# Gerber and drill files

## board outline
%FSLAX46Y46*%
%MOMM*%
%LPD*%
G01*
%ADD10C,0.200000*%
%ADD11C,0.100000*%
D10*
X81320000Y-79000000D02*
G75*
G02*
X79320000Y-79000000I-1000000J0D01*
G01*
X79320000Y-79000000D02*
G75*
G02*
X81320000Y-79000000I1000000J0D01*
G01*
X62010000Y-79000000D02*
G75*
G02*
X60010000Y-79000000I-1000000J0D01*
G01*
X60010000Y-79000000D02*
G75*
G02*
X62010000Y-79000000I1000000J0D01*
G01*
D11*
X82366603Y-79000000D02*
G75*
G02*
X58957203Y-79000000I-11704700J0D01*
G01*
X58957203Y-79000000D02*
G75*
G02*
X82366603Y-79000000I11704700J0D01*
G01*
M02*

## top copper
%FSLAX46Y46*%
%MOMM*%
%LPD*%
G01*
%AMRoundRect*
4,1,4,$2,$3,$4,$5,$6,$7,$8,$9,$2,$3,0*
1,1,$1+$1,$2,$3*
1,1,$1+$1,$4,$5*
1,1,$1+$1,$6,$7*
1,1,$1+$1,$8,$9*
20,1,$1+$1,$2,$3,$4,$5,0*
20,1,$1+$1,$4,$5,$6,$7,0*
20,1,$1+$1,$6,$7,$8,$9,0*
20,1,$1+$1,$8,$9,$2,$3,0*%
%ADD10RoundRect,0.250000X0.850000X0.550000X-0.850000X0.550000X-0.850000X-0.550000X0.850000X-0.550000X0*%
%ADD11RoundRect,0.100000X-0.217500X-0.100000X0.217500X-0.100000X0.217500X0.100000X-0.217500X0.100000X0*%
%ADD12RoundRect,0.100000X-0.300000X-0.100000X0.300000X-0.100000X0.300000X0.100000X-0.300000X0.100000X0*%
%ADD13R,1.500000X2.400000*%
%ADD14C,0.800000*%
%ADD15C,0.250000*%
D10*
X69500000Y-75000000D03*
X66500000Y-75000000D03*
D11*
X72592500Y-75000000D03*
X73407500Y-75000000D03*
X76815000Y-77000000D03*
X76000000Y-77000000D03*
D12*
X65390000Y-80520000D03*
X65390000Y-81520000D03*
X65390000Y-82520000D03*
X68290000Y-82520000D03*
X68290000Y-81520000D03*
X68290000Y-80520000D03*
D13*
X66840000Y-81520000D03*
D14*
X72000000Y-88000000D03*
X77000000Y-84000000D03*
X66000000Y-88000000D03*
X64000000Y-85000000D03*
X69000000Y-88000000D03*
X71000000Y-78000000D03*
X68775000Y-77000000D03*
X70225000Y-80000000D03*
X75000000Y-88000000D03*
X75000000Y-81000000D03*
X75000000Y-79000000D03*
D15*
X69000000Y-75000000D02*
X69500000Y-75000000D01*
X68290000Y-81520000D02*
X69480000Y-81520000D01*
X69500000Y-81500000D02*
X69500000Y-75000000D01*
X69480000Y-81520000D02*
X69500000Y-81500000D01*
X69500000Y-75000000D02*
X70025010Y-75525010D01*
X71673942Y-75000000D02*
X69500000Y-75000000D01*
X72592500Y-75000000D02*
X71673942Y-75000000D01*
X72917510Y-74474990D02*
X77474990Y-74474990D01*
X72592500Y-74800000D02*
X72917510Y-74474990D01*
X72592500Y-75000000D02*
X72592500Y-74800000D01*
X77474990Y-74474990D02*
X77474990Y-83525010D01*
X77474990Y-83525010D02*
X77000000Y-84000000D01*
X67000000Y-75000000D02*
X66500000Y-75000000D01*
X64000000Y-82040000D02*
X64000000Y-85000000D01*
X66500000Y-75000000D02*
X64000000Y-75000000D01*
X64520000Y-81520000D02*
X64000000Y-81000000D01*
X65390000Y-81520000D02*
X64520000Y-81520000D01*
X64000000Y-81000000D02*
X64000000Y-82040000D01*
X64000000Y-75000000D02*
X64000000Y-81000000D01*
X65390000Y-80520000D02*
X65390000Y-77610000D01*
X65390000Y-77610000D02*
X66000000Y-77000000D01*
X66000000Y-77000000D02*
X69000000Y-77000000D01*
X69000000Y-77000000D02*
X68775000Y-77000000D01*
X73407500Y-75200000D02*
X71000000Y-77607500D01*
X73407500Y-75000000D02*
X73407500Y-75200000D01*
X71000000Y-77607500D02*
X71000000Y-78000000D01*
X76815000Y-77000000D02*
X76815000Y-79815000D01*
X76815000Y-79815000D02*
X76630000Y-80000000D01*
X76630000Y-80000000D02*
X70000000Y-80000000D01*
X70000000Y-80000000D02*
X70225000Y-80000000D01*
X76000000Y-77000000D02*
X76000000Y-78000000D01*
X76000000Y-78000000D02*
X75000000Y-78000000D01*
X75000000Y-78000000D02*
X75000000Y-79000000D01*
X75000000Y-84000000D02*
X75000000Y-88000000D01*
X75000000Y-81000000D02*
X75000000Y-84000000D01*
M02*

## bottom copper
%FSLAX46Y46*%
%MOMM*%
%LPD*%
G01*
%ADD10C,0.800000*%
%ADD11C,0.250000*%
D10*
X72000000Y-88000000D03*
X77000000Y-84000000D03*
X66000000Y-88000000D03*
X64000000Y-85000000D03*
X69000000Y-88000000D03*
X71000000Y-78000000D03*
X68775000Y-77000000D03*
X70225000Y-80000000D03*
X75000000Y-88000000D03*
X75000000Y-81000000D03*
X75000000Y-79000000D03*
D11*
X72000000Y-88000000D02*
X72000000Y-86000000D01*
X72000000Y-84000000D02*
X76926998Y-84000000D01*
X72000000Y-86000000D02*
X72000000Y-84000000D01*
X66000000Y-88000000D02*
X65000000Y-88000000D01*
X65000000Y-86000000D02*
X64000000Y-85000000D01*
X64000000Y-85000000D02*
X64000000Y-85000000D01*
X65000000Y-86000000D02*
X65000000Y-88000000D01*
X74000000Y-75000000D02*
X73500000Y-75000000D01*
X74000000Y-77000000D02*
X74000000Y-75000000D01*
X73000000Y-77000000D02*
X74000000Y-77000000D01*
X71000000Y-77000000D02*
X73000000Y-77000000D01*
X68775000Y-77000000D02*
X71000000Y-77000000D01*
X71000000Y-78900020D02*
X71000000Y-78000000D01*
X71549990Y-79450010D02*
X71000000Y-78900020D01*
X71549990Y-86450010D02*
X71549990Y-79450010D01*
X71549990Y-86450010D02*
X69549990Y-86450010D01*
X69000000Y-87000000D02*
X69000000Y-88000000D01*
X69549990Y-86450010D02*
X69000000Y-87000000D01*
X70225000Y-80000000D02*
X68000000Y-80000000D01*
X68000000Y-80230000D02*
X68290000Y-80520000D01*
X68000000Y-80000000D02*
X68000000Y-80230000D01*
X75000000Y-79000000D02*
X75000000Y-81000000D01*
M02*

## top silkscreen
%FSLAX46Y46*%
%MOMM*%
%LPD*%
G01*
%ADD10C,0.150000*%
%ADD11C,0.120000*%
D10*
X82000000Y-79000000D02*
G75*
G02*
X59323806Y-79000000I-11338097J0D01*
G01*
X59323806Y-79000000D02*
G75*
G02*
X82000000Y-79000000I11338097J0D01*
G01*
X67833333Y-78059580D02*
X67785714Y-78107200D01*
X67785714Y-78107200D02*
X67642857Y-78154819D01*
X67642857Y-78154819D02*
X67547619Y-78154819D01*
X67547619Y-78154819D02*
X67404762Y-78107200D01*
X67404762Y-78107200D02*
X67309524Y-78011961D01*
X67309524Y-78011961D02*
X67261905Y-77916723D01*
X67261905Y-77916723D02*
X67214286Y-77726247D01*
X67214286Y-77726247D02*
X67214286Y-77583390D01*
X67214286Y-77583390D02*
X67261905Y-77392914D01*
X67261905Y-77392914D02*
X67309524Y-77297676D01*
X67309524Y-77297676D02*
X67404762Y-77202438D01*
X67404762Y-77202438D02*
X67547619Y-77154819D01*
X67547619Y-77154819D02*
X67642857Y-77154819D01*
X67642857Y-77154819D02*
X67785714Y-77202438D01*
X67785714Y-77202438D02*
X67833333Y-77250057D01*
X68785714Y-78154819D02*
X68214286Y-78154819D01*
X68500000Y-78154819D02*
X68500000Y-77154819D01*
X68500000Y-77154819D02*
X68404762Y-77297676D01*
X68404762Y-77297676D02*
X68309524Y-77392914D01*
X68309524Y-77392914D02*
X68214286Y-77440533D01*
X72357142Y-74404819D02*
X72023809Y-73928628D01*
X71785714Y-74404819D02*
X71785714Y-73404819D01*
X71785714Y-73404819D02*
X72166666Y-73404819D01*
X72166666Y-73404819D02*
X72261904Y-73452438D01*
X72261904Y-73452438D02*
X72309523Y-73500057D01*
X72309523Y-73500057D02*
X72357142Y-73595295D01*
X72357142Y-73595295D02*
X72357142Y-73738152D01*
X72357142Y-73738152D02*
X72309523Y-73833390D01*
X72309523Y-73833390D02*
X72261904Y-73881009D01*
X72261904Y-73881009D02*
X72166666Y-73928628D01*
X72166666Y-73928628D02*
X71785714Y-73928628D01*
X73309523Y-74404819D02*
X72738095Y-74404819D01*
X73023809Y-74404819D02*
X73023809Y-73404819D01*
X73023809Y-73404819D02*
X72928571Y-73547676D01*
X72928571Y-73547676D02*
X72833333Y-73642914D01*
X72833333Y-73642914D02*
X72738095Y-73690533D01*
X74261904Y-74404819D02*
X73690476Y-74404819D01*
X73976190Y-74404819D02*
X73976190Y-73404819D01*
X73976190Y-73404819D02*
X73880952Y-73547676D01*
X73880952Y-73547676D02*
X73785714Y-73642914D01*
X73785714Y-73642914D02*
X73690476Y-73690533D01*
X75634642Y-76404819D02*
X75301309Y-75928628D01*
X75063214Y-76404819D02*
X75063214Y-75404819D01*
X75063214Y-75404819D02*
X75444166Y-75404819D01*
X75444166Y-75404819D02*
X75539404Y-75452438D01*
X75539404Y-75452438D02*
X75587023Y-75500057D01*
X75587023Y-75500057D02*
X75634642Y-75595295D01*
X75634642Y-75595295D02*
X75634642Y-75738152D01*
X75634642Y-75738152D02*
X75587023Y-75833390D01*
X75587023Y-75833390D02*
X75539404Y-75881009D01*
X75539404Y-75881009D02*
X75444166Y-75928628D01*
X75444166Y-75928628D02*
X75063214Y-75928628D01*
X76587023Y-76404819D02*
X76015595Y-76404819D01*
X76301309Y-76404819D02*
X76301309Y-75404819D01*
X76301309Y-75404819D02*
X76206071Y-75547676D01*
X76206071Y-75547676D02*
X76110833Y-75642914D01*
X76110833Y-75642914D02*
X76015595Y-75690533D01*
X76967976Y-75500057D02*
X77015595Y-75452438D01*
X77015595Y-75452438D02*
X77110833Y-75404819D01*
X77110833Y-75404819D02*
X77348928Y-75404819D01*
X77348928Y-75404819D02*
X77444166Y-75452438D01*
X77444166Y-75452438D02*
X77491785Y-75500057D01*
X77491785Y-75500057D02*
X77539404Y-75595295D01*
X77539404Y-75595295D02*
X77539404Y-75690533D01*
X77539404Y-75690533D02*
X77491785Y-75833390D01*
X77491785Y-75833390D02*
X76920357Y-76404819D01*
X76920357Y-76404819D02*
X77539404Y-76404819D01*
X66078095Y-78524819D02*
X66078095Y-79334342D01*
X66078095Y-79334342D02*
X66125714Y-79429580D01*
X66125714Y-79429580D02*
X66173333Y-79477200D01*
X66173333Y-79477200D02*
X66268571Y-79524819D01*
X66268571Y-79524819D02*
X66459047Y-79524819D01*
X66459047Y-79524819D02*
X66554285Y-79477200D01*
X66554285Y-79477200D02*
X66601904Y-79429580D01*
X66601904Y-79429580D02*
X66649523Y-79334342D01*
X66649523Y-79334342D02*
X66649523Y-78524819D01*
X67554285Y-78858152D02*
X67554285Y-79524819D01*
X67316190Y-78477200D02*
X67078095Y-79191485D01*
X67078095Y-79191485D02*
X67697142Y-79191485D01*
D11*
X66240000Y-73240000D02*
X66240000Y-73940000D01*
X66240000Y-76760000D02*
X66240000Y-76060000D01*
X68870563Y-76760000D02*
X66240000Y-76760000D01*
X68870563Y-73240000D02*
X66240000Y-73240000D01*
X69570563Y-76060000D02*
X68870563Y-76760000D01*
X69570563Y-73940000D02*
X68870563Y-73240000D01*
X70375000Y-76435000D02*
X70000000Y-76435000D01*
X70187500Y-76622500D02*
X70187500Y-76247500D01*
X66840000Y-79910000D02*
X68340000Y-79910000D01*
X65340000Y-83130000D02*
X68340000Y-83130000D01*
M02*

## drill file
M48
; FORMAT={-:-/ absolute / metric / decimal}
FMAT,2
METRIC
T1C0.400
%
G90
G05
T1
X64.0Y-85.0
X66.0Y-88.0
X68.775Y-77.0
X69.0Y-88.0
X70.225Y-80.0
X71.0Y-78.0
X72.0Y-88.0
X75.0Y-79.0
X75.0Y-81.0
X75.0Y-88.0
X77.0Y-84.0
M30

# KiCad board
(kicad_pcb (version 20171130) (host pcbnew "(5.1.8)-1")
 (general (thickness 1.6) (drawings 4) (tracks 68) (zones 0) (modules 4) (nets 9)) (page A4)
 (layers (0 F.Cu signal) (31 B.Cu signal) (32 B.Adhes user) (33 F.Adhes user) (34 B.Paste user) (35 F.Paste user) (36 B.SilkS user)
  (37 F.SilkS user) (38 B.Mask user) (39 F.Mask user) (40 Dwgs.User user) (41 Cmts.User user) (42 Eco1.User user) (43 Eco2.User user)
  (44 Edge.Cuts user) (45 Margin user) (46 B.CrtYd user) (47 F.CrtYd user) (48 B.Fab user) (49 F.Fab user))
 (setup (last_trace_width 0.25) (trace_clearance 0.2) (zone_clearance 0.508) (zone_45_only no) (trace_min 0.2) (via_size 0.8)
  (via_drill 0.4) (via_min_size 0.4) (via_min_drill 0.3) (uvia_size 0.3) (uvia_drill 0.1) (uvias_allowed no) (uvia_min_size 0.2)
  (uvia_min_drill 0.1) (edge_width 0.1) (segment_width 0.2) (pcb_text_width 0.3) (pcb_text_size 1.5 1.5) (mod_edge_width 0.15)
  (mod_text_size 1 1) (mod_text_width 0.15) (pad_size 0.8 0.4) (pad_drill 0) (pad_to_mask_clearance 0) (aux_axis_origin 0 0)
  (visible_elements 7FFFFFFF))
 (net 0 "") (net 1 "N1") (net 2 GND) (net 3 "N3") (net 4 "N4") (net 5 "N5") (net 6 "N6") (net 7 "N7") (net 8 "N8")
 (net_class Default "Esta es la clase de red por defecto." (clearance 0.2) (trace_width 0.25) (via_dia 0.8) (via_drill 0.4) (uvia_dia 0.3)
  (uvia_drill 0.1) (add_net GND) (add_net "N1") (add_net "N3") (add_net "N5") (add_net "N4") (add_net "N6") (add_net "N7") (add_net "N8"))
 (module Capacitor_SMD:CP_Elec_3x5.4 (layer F.Cu) (at 68 75 180)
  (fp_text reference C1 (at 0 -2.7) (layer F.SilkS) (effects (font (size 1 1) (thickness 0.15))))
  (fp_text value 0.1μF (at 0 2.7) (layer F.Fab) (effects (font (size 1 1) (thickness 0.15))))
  (fp_line (start 1.76 1.76) (end 1.76 1.06) (layer F.SilkS) (width 0.12))
  (fp_line (start 1.76 -1.76) (end 1.76 -1.06) (layer F.SilkS) (width 0.12))
  (fp_line (start -0.870563 -1.76) (end 1.76 -1.76) (layer F.SilkS) (width 0.12))
  (fp_line (start -0.870563 1.76) (end 1.76 1.76) (layer F.SilkS) (width 0.12))
  (fp_line (start -1.570563 -1.06) (end -0.870563 -1.76) (layer F.SilkS) (width 0.12))
  (fp_line (start -1.570563 1.06) (end -0.870563 1.76) (layer F.SilkS) (width 0.12))
  (fp_line (start -2.375 -1.435) (end -2 -1.435) (layer F.SilkS) (width 0.12))
  (fp_line (start -2.1875 -1.6225) (end -2.1875 -1.2475) (layer F.SilkS) (width 0.12))
  (pad 1 smd roundrect (at -1.5 0 180) (size 2.2 1.6) (layers F.Cu F.Paste F.Mask) (roundrect_rratio 0.15625) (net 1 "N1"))
  (pad 2 smd roundrect (at 1.5 0 180) (size 2.2 1.6) (layers F.Cu F.Paste F.Mask) (roundrect_rratio 0.15625) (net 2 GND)))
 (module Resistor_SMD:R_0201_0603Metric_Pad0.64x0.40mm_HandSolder (layer F.Cu) (at 73 75)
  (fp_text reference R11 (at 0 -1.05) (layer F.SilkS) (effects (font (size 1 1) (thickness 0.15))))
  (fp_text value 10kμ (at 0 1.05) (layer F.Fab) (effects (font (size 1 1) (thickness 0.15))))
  (pad "" smd roundrect (at -0.4325 0) (size 0.458 0.36) (layers F.Paste) (roundrect_rratio 0.25))
  (pad "" smd roundrect (at 0.4325 0) (size 0.458 0.36) (layers F.Paste) (roundrect_rratio 0.25))
  (pad 1 smd roundrect (at -0.4075 0) (size 0.635 0.4) (layers F.Cu F.Mask) (roundrect_rratio 0.25) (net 1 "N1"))
  (pad 2 smd roundrect (at 0.4075 0) (size 0.635 0.4) (layers F.Cu F.Mask) (roundrect_rratio 0.25) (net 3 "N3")))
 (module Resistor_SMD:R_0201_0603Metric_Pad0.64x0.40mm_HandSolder (layer F.Cu) (at 76.4075 77)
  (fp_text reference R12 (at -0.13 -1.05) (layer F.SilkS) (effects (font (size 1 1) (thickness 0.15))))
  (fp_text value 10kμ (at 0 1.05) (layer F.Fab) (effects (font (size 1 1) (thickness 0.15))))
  (pad 2 smd roundrect (at 0.4075 0) (size 0.635 0.4) (layers F.Cu F.Mask) (roundrect_rratio 0.25) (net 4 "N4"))
  (pad 1 smd roundrect (at -0.4075 0) (size 0.635 0.4) (layers F.Cu F.Mask) (roundrect_rratio 0.25) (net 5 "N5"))
  (pad "" smd roundrect (at 0.4325 0) (size 0.458 0.36) (layers F.Paste) (roundrect_rratio 0.25))
  (pad "" smd roundrect (at -0.4325 0) (size 0.458 0.36) (layers F.Paste) (roundrect_rratio 0.25)))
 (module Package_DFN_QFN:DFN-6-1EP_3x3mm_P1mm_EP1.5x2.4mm (layer F.Cu) (at 66.84 81.52)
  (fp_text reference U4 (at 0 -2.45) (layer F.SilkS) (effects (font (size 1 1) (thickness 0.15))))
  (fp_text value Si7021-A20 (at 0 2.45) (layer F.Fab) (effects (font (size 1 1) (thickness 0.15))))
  (fp_line (start 0 -1.61) (end 1.5 -1.61) (layer F.SilkS) (width 0.12))
  (fp_line (start -1.5 1.61) (end 1.5 1.61) (layer F.SilkS) (width 0.12))
  (pad SDA smd roundrect (at -1.45 -1) (size 0.8 0.4) (layers F.Cu F.Paste F.Mask) (roundrect_rratio 0.25) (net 3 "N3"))
  (pad 2 smd roundrect (at -1.45 0) (size 0.8 0.4) (layers F.Cu F.Paste F.Mask) (roundrect_rratio 0.25) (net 2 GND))
  (pad DNC smd roundrect (at -1.45 1) (size 0.8 0.4) (layers F.Cu F.Paste F.Mask) (roundrect_rratio 0.25) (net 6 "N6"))
  (pad DNC smd roundrect (at 1.45 1) (size 0.8 0.4) (layers F.Cu F.Paste F.Mask) (roundrect_rratio 0.25) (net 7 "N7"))
  (pad VDD smd roundrect (at 1.45 0) (size 0.8 0.4) (layers F.Cu F.Paste F.Mask) (roundrect_rratio 0.25) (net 1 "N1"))
  (pad SCL smd roundrect (at 1.45 -1) (size 0.8 0.4) (layers F.Cu F.Paste F.Mask) (roundrect_rratio 0.25) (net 4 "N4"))
  (pad 7 smd rect (at 0 0) (size 1.5 2.4) (layers F.Cu F.Mask) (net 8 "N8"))
  (pad "" smd roundrect (at -0.375 -0.6) (size 0.6 0.97) (layers F.Paste) (roundrect_rratio 0.25))
  (pad "" smd roundrect (at -0.375 0.6) (size 0.6 0.97) (layers F.Paste) (roundrect_rratio 0.25))
  (pad "" smd roundrect (at 0.375 -0.6) (size 0.6 0.97) (layers F.Paste) (roundrect_rratio 0.25))
  (pad "" smd roundrect (at 0.375 0.6) (size 0.6 0.97) (layers F.Paste) (roundrect_rratio 0.25)))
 (gr_circle (center 80.32 79) (end 81.32 79) (layer Edge.Cuts) (width 0.2))
 (gr_circle (center 61.01 79) (end 62.01 79) (layer Edge.Cuts) (width 0.2))
 (gr_circle (center 70.661903 79) (end 82 79) (layer F.SilkS) (width 0.15))
 (gr_circle (center 70.661903 79) (end 82.366603 79) (layer Edge.Cuts) (width 0.1))
 (via (at 72 88) (size 0.8) (drill 0.4) (layers F.Cu B.Cu) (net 1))
 (segment (start 72 88) (end 72 86) (width 0.25) (layer B.Cu) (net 1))
 (segment (start 72 84) (end 76.926998 84) (width 0.25) (layer B.Cu) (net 1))
 (via (at 77 84) (size 0.8) (drill 0.4) (layers F.Cu B.Cu) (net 1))
 (segment (start 69 75) (end 69.5 75) (width 0.25) (layer F.Cu) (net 1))
 (segment (start 68.29 81.52) (end 69.48 81.52) (width 0.25) (layer F.Cu) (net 1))
 (segment (start 69.5 81.5) (end 69.5 75) (width 0.25) (layer F.Cu) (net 1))
 (segment (start 69.48 81.52) (end 69.5 81.5) (width 0.25) (layer F.Cu) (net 1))
 (segment (start 69.5 75) (end 70.02501 75.52501) (width 0.25) (layer F.Cu) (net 1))
 (segment (start 71.673942 75) (end 69.5 75) (width 0.25) (layer F.Cu) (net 1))
 (segment (start 72.5925 75) (end 71.673942 75) (width 0.25) (layer F.Cu) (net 1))
 (segment (start 72.91751 74.47499) (end 77.47499 74.47499) (width 0.25) (layer F.Cu) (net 1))
 (segment (start 72.5925 74.8) (end 72.91751 74.47499) (width 0.25) (layer F.Cu) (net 1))
 (segment (start 72.5925 75) (end 72.5925 74.8) (width 0.25) (layer F.Cu) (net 1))
 (segment (start 77.47499 74.47499) (end 77.47499 83.52501) (width 0.25) (layer F.Cu) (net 1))
 (segment (start 77.47499 83.52501) (end 77 84) (width 0.25) (layer F.Cu) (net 1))
 (segment (start 72 86) (end 72 84) (width 0.25) (layer B.Cu) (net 1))
 (via (at 66 88) (size 0.8) (drill 0.4) (layers F.Cu B.Cu) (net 2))
 (segment (start 66 88) (end 65 88) (width 0.25) (layer B.Cu) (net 2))
 (segment (start 65 86) (end 64 85) (width 0.25) (layer B.Cu) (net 2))
 (segment (start 64 85) (end 64 85) (width 0.25) (layer B.Cu) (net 2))
 (via (at 64 85) (size 0.8) (drill 0.4) (layers F.Cu B.Cu) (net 2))
 (segment (start 67 75) (end 66.5 75) (width 0.25) (layer F.Cu) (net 2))
 (segment (start 64 82.04) (end 64 85) (width 0.25) (layer F.Cu) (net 2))
 (segment (start 66.5 75) (end 64 75) (width 0.25) (layer F.Cu) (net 2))
 (segment (start 64.52 81.52) (end 64 81) (width 0.25) (layer F.Cu) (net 2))
 (segment (start 65.39 81.52) (end 64.52 81.52) (width 0.25) (layer F.Cu) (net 2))
 (segment (start 64 81) (end 64 82.04) (width 0.25) (layer F.Cu) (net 2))
 (segment (start 64 75) (end 64 81) (width 0.25) (layer F.Cu) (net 2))
 (segment (start 65 86) (end 65 88) (width 0.25) (layer B.Cu) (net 2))
 (via (at 69 88) (size 0.8) (drill 0.4) (layers F.Cu B.Cu) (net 3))
 (via (at 71 78) (size 0.8) (drill 0.4) (layers F.Cu B.Cu) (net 3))
 (segment (start 65.39 80.52) (end 65.39 77.61) (width 0.25) (layer F.Cu) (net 3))
 (segment (start 65.39 77.61) (end 66 77) (width 0.25) (layer F.Cu) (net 3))
 (segment (start 66 77) (end 69 77) (width 0.25) (layer F.Cu) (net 3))
 (via (at 68.775 77) (size 0.8) (drill 0.4) (layers F.Cu B.Cu) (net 3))
 (segment (start 69 77) (end 68.775 77) (width 0.25) (layer F.Cu) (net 3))
 (segment (start 74 75) (end 73.5 75) (width 0.25) (layer B.Cu) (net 3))
 (segment (start 74 77) (end 74 75) (width 0.25) (layer B.Cu) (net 3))
 (segment (start 73 77) (end 74 77) (width 0.25) (layer B.Cu) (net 3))
 (segment (start 71 77) (end 73 77) (width 0.25) (layer B.Cu) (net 3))
 (segment (start 68.775 77) (end 71 77) (width 0.25) (layer B.Cu) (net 3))
 (segment (start 73.4075 75.2) (end 71 77.6075) (width 0.25) (layer F.Cu) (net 3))
 (segment (start 73.4075 75) (end 73.4075 75.2) (width 0.25) (layer F.Cu) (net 3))
 (segment (start 71 77.6075) (end 71 78) (width 0.25) (layer F.Cu) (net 3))
 (segment (start 71 78.90002) (end 71 78) (width 0.25) (layer B.Cu) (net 3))
 (segment (start 71.54999 79.45001) (end 71 78.90002) (width 0.25) (layer B.Cu) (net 3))
 (segment (start 71.54999 86.45001) (end 71.54999 79.45001) (width 0.25) (layer B.Cu) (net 3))
 (segment (start 71.54999 86.45001) (end 69.54999 86.45001) (width 0.25) (layer B.Cu) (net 3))
 (segment (start 69 87) (end 69 88) (width 0.25) (layer B.Cu) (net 3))
 (segment (start 69.54999 86.45001) (end 69 87) (width 0.25) (layer B.Cu) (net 3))
 (segment (start 76.815 77) (end 76.815 79.815) (width 0.25) (layer F.Cu) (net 4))
 (segment (start 76.815 79.815) (end 76.63 80) (width 0.25) (layer F.Cu) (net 4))
 (segment (start 76.63 80) (end 70 80) (width 0.25) (layer F.Cu) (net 4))
 (via (at 70.225 80) (size 0.8) (drill 0.4) (layers F.Cu B.Cu) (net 4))
 (segment (start 70 80) (end 70.225 80) (width 0.25) (layer F.Cu) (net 4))
 (segment (start 70.225 80) (end 68 80) (width 0.25) (layer B.Cu) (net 4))
 (segment (start 68 80.23) (end 68.29 80.52) (width 0.25) (layer B.Cu) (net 4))
 (segment (start 68 80) (end 68 80.23) (width 0.25) (layer B.Cu) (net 4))
 (via (at 75 88) (size 0.8) (drill 0.4) (layers F.Cu B.Cu) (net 5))
 (via (at 75 81) (size 0.8) (drill 0.4) (layers F.Cu B.Cu) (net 5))
 (segment (start 76 77) (end 76 78) (width 0.25) (layer F.Cu) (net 5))
 (segment (start 76 78) (end 75 78) (width 0.25) (layer F.Cu) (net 5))
 (segment (start 75 78) (end 75 79) (width 0.25) (layer F.Cu) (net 5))
 (via (at 75 79) (size 0.8) (drill 0.4) (layers F.Cu B.Cu) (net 5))
 (segment (start 75 79) (end 75 81) (width 0.25) (layer B.Cu) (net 5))
 (segment (start 75 84) (end 75 88) (width 0.25) (layer F.Cu) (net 5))
 (segment (start 75 81) (end 75 84) (width 0.25) (layer F.Cu) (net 5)))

